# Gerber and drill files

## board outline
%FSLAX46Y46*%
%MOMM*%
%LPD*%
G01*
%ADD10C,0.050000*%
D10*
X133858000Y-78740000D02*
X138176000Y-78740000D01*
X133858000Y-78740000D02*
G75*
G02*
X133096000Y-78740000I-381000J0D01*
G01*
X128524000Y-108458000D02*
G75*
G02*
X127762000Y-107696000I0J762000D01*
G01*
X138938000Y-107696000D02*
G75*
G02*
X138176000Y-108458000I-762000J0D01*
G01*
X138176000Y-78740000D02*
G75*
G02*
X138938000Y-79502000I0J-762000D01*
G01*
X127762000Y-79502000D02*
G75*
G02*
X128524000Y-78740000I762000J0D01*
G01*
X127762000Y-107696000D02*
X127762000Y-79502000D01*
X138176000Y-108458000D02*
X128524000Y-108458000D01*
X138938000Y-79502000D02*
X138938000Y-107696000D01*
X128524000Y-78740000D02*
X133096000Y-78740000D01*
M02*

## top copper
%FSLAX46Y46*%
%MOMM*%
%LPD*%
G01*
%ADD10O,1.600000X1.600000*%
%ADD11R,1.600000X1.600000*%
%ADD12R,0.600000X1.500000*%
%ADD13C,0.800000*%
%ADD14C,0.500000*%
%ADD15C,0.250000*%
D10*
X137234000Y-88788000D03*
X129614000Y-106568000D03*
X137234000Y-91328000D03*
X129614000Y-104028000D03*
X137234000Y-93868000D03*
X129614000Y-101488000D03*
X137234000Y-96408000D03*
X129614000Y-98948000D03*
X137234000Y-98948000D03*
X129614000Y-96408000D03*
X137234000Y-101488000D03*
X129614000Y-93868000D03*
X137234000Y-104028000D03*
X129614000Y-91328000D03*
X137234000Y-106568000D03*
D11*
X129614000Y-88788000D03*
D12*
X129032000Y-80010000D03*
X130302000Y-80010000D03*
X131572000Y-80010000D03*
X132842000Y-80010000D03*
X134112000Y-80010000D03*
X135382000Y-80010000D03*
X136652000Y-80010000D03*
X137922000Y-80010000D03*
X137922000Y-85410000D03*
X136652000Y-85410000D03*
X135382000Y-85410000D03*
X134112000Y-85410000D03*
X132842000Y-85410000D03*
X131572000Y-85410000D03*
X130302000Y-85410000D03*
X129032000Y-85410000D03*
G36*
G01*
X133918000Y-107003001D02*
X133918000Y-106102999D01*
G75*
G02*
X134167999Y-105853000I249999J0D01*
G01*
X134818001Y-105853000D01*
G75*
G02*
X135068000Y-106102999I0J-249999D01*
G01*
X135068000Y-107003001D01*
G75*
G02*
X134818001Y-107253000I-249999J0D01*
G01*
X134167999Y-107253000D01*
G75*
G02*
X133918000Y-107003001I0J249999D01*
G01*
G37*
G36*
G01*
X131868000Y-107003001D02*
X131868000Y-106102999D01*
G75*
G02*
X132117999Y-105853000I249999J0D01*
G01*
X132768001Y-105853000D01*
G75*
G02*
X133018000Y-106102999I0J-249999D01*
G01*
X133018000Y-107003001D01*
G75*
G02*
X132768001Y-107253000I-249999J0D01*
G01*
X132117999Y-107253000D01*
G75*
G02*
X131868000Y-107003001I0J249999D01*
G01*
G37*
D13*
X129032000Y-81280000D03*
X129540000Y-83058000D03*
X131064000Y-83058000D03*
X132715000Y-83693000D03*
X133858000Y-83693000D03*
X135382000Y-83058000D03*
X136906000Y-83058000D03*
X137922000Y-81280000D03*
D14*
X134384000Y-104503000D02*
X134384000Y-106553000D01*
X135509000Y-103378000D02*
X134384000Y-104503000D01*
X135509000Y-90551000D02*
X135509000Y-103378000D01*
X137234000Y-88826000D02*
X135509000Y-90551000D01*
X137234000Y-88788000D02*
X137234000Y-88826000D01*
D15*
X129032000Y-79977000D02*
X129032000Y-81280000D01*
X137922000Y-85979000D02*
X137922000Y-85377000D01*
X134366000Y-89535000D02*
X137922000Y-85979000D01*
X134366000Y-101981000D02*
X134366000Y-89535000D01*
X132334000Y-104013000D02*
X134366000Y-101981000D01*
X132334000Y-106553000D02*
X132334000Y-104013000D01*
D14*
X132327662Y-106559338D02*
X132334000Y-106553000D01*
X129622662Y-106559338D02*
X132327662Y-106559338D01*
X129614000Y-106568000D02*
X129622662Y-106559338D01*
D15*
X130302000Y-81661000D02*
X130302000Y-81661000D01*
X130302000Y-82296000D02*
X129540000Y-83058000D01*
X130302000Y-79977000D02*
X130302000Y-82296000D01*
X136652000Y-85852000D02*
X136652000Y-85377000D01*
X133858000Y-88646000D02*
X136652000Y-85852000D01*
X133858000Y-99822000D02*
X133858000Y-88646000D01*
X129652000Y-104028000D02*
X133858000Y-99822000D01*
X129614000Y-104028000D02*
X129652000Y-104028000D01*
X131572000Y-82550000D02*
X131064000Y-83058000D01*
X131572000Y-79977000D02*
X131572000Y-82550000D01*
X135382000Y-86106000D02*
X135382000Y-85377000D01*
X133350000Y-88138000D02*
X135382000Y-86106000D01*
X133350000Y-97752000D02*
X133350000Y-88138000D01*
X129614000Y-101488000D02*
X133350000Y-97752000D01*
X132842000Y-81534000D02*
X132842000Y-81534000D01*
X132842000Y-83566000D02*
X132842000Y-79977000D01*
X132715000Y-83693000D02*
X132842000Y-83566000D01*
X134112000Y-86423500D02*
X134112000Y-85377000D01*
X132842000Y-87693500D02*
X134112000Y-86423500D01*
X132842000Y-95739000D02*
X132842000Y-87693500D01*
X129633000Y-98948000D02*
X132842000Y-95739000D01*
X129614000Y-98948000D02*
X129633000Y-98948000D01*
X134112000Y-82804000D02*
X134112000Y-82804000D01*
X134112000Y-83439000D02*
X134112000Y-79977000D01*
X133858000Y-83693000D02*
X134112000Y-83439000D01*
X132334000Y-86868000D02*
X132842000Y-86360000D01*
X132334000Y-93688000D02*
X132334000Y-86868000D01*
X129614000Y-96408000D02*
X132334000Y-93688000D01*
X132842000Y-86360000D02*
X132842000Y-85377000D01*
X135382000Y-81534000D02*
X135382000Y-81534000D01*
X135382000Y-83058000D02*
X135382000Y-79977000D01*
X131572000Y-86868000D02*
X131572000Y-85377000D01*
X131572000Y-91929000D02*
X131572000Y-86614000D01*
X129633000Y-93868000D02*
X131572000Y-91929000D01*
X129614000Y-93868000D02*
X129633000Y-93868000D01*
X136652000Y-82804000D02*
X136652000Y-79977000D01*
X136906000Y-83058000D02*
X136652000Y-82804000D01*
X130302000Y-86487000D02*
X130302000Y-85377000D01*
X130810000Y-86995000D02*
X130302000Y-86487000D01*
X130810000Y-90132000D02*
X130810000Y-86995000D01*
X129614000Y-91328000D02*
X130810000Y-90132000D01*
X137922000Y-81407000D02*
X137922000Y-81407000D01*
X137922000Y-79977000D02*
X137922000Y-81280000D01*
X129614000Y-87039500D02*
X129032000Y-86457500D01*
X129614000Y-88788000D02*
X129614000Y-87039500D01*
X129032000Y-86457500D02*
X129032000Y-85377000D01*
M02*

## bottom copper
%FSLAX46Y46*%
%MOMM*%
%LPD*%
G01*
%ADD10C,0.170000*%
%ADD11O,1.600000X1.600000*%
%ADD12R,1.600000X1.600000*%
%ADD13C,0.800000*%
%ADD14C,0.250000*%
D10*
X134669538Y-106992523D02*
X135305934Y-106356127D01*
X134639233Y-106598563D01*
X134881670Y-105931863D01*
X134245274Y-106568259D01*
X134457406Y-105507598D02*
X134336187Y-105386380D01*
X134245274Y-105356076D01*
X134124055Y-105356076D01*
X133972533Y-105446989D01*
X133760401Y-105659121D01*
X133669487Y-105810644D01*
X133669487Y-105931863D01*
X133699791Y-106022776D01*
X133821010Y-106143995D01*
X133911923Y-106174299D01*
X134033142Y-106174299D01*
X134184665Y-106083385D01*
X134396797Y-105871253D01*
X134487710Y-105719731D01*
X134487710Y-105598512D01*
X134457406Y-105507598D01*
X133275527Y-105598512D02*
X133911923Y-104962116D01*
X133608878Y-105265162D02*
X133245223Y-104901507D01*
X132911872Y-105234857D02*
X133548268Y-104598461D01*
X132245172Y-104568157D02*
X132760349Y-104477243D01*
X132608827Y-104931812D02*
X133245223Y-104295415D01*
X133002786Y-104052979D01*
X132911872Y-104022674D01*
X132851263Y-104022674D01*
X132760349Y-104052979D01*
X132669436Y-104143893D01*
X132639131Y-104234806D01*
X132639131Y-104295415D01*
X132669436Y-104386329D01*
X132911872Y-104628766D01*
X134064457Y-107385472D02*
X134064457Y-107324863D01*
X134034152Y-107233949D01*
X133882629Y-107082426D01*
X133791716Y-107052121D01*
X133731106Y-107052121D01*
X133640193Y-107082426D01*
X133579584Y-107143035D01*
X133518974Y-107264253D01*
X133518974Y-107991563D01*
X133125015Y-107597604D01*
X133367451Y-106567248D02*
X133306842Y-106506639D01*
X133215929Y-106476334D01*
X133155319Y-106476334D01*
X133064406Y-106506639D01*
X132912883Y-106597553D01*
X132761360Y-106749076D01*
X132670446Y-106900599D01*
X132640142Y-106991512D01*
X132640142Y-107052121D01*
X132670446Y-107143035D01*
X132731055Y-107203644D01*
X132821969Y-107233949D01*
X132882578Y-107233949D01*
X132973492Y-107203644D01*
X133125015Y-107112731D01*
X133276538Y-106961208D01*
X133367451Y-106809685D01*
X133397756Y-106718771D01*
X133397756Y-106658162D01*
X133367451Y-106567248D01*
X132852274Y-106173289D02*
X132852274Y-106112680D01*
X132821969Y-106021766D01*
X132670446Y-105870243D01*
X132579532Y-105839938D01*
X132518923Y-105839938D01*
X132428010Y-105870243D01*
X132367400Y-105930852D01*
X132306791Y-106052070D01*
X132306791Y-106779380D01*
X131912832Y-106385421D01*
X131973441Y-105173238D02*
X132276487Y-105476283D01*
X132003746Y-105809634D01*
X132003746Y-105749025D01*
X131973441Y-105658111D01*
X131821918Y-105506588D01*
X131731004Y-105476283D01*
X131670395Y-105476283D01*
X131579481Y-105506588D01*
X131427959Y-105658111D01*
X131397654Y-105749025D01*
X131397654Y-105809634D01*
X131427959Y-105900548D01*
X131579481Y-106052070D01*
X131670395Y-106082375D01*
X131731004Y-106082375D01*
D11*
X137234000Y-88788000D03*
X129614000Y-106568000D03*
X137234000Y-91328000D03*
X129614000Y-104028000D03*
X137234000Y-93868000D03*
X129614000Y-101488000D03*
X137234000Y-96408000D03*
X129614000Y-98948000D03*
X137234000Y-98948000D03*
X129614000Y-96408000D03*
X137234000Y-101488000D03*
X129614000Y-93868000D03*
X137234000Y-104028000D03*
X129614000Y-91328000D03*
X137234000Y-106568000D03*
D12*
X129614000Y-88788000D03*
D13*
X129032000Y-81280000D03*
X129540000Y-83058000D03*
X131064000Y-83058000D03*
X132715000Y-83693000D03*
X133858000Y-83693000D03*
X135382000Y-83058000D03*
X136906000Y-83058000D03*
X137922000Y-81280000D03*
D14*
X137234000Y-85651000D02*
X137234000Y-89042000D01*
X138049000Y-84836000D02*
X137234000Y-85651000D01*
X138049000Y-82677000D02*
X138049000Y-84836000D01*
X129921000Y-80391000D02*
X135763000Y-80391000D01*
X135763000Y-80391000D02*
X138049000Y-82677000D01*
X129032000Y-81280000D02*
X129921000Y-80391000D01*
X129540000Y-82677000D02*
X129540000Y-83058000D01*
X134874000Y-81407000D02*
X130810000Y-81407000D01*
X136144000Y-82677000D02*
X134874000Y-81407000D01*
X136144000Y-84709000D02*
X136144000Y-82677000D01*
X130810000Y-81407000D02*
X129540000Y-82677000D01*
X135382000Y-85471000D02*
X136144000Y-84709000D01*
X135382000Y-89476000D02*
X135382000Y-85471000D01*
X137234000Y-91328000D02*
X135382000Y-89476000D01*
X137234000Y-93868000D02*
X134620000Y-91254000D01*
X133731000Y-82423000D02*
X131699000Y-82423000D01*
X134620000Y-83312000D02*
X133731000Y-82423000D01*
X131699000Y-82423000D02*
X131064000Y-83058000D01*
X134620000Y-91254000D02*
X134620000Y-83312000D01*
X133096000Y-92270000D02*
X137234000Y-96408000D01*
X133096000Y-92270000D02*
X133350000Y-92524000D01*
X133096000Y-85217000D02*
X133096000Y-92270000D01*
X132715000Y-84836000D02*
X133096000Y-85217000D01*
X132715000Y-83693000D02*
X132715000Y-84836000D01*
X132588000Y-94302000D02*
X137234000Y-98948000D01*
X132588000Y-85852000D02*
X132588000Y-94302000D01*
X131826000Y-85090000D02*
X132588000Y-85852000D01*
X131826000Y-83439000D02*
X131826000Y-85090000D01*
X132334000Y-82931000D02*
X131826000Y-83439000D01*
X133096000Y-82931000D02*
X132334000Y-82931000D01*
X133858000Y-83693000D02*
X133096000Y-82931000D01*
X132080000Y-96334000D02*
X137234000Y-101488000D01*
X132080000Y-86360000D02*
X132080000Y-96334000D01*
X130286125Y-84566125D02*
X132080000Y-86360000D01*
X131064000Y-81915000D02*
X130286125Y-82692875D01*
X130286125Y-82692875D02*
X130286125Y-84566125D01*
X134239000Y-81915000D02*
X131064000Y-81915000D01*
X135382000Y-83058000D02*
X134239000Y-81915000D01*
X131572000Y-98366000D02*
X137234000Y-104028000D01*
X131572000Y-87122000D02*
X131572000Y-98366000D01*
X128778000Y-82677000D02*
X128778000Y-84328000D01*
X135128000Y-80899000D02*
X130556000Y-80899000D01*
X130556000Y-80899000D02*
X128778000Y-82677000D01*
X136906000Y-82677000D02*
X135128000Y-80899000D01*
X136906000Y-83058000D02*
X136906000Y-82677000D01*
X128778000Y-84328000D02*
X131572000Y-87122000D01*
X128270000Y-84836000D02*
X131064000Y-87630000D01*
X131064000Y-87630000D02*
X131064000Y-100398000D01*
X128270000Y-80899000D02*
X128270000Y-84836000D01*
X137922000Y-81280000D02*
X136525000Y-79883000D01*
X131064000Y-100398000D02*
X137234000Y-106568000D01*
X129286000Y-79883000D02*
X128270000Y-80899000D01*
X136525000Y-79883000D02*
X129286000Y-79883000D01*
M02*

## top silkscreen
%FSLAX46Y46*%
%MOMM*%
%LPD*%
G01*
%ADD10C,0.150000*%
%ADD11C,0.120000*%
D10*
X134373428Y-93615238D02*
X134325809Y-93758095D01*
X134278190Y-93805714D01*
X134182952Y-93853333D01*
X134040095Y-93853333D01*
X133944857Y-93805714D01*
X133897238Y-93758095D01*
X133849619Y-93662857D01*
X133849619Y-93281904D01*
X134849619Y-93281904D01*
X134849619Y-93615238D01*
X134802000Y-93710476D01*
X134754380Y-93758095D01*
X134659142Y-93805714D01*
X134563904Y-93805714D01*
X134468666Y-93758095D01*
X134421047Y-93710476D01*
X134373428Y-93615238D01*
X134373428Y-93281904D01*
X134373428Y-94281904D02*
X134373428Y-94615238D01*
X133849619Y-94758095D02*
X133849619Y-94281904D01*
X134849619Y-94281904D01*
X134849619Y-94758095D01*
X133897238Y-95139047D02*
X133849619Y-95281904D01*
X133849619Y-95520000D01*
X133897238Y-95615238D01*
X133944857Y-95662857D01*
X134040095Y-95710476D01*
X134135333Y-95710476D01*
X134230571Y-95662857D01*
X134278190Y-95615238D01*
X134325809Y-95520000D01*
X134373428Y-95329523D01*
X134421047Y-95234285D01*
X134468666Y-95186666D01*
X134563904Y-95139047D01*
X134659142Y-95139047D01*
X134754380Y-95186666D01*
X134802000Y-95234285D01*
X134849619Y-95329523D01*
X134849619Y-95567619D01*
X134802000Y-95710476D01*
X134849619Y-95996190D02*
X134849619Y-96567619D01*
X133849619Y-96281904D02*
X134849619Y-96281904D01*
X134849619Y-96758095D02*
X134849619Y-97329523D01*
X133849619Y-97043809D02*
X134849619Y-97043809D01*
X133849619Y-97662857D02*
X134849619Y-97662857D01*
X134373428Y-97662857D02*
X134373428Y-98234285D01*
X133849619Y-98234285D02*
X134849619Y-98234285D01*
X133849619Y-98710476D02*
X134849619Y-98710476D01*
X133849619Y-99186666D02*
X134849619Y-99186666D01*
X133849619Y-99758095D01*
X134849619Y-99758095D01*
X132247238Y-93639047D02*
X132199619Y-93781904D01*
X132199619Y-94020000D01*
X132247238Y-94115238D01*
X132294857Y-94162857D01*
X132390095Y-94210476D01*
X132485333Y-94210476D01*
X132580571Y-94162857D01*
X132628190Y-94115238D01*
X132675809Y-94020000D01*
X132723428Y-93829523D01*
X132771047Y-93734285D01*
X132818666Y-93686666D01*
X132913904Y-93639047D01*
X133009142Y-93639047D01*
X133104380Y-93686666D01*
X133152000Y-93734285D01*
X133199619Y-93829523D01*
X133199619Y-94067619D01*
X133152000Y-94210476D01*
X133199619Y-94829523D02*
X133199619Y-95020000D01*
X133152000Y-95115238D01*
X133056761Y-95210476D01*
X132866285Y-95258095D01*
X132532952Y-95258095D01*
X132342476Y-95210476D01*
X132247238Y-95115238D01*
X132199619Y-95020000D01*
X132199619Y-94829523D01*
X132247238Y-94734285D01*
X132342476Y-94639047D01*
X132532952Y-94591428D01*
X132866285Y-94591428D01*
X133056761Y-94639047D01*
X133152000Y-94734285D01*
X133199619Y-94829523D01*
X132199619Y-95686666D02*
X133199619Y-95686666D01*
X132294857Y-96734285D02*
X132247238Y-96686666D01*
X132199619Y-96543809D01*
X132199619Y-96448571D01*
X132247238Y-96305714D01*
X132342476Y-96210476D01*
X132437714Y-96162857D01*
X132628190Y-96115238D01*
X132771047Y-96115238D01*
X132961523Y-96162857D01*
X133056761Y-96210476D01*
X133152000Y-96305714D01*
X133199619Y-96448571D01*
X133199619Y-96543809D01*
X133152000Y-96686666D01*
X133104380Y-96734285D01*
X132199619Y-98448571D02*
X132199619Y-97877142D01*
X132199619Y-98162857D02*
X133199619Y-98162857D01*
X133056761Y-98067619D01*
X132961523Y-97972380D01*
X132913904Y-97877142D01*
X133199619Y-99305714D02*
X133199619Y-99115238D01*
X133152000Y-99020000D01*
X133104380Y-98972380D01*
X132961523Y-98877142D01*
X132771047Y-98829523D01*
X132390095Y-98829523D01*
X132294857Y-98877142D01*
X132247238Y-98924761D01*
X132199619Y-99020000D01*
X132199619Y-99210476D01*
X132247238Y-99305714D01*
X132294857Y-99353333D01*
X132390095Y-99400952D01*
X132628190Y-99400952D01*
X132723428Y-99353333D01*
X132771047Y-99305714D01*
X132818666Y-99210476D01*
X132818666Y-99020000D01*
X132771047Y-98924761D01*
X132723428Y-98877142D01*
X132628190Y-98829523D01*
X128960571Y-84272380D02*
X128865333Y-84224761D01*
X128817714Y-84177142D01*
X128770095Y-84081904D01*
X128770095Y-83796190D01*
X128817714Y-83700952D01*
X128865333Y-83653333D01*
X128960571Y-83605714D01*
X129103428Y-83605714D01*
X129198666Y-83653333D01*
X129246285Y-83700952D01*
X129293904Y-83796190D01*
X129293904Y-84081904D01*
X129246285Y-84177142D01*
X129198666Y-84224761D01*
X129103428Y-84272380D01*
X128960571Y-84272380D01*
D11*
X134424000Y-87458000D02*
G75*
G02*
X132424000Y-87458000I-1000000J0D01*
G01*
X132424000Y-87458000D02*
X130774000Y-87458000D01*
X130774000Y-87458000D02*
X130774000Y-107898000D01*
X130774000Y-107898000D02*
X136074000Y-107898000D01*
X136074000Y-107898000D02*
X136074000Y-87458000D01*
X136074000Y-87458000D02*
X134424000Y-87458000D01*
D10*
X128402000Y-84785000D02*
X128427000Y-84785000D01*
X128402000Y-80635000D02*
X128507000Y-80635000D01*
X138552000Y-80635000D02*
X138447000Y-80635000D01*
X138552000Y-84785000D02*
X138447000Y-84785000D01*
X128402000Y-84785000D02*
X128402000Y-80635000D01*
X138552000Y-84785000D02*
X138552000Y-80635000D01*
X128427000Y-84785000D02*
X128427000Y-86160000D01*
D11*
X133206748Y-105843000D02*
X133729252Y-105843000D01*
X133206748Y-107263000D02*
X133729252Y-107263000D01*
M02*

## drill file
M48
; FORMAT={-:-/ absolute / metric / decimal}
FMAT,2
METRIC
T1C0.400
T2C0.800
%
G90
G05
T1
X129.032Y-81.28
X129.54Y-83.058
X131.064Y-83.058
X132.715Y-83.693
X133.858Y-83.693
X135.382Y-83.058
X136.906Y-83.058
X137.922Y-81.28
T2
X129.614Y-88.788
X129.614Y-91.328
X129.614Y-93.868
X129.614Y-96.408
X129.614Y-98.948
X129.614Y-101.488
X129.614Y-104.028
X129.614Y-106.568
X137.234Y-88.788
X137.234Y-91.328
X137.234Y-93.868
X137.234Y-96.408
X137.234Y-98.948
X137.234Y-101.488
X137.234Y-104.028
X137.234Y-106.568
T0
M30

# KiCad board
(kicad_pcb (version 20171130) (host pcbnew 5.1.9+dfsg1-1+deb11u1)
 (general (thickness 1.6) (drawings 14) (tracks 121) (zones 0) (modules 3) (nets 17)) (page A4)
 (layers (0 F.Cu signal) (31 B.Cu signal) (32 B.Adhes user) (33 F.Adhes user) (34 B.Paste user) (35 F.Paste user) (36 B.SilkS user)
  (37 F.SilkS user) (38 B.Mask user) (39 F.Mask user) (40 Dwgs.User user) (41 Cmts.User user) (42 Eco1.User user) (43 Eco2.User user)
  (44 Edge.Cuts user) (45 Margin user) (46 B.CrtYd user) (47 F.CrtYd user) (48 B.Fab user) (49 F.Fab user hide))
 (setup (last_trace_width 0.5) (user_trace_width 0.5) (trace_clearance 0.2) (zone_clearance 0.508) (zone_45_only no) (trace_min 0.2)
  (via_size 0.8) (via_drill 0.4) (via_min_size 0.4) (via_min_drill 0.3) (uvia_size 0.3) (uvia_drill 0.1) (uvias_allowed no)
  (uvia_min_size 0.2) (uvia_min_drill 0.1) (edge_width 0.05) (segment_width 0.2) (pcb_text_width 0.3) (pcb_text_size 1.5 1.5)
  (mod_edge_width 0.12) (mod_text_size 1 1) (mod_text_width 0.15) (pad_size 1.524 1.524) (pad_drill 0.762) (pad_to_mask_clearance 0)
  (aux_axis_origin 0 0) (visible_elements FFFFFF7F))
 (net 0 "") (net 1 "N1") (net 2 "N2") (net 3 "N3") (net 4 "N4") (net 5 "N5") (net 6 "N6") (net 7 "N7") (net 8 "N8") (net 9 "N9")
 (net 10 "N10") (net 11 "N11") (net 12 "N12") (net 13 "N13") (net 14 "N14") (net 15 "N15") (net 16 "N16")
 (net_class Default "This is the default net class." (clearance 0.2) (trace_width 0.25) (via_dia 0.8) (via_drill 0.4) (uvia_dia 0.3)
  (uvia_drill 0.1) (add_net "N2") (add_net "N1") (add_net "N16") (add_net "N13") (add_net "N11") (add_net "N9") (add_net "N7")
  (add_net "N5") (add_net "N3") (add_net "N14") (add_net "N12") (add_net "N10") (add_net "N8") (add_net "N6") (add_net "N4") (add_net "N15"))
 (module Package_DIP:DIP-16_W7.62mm (layer F.Cu) (at 129.614 88.788)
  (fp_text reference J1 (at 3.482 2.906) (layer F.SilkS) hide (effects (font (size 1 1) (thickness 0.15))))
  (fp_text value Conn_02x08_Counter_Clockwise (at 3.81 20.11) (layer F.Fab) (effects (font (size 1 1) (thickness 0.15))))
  (fp_arc (start 3.81 -1.33) (end 2.81 -1.33) (angle -180) (layer F.SilkS) (width 0.12))
  (fp_line (start 2.81 -1.33) (end 1.16 -1.33) (layer F.SilkS) (width 0.12))
  (fp_line (start 1.16 -1.33) (end 1.16 19.11) (layer F.SilkS) (width 0.12))
  (fp_line (start 1.16 19.11) (end 6.46 19.11) (layer F.SilkS) (width 0.12))
  (fp_line (start 6.46 19.11) (end 6.46 -1.33) (layer F.SilkS) (width 0.12))
  (fp_line (start 6.46 -1.33) (end 4.81 -1.33) (layer F.SilkS) (width 0.12))
  (pad 16 thru_hole oval (at 7.62 0) (size 1.6 1.6) (drill 0.8) (layers *.Cu *.Mask) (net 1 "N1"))
  (pad 8 thru_hole oval (at 0 17.78) (size 1.6 1.6) (drill 0.8) (layers *.Cu *.Mask) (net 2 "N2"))
  (pad 15 thru_hole oval (at 7.62 2.54) (size 1.6 1.6) (drill 0.8) (layers *.Cu *.Mask) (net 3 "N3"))
  (pad 7 thru_hole oval (at 0 15.24) (size 1.6 1.6) (drill 0.8) (layers *.Cu *.Mask) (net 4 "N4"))
  (pad 14 thru_hole oval (at 7.62 5.08) (size 1.6 1.6) (drill 0.8) (layers *.Cu *.Mask) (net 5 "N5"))
  (pad 6 thru_hole oval (at 0 12.7) (size 1.6 1.6) (drill 0.8) (layers *.Cu *.Mask) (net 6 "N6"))
  (pad 13 thru_hole oval (at 7.62 7.62) (size 1.6 1.6) (drill 0.8) (layers *.Cu *.Mask) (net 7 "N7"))
  (pad 5 thru_hole oval (at 0 10.16) (size 1.6 1.6) (drill 0.8) (layers *.Cu *.Mask) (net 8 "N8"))
  (pad 12 thru_hole oval (at 7.62 10.16) (size 1.6 1.6) (drill 0.8) (layers *.Cu *.Mask) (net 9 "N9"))
  (pad 4 thru_hole oval (at 0 7.62) (size 1.6 1.6) (drill 0.8) (layers *.Cu *.Mask) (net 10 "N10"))
  (pad 11 thru_hole oval (at 7.62 12.7) (size 1.6 1.6) (drill 0.8) (layers *.Cu *.Mask) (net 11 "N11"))
  (pad 3 thru_hole oval (at 0 5.08) (size 1.6 1.6) (drill 0.8) (layers *.Cu *.Mask) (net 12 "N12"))
  (pad 10 thru_hole oval (at 7.62 15.24) (size 1.6 1.6) (drill 0.8) (layers *.Cu *.Mask) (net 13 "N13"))
  (pad 2 thru_hole oval (at 0 2.54) (size 1.6 1.6) (drill 0.8) (layers *.Cu *.Mask) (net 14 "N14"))
  (pad 9 thru_hole oval (at 7.62 17.78) (size 1.6 1.6) (drill 0.8) (layers *.Cu *.Mask) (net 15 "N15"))
  (pad 1 thru_hole rect (at 0 0) (size 1.6 1.6) (drill 0.8) (layers *.Cu *.Mask) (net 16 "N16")))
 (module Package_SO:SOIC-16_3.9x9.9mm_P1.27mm (layer F.Cu) (at 133.477 82.71 90)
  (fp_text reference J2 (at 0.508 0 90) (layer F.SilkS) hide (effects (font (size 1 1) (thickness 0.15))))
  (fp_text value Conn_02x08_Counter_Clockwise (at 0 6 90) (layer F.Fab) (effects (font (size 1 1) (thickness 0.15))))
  (fp_line (start -2.075 -5.075) (end -2.075 -5.05) (layer F.SilkS) (width 0.15))
  (fp_line (start 2.075 -5.075) (end 2.075 -4.97) (layer F.SilkS) (width 0.15))
  (fp_line (start 2.075 5.075) (end 2.075 4.97) (layer F.SilkS) (width 0.15))
  (fp_line (start -2.075 5.075) (end -2.075 4.97) (layer F.SilkS) (width 0.15))
  (fp_line (start -2.075 -5.075) (end 2.075 -5.075) (layer F.SilkS) (width 0.15))
  (fp_line (start -2.075 5.075) (end 2.075 5.075) (layer F.SilkS) (width 0.15))
  (fp_line (start -2.075 -5.05) (end -3.45 -5.05) (layer F.SilkS) (width 0.15))
  (pad 16 smd rect (at 2.7 -4.445 90) (size 1.5 0.6) (layers F.Cu F.Paste F.Mask) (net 1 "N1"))
  (pad 15 smd rect (at 2.7 -3.175 90) (size 1.5 0.6) (layers F.Cu F.Paste F.Mask) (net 3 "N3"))
  (pad 14 smd rect (at 2.7 -1.905 90) (size 1.5 0.6) (layers F.Cu F.Paste F.Mask) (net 5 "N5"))
  (pad 13 smd rect (at 2.7 -0.635 90) (size 1.5 0.6) (layers F.Cu F.Paste F.Mask) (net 7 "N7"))
  (pad 12 smd rect (at 2.7 0.635 90) (size 1.5 0.6) (layers F.Cu F.Paste F.Mask) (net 9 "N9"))
  (pad 11 smd rect (at 2.7 1.905 90) (size 1.5 0.6) (layers F.Cu F.Paste F.Mask) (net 11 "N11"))
  (pad 10 smd rect (at 2.7 3.175 90) (size 1.5 0.6) (layers F.Cu F.Paste F.Mask) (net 13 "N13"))
  (pad 9 smd rect (at 2.7 4.445 90) (size 1.5 0.6) (layers F.Cu F.Paste F.Mask) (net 15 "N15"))
  (pad 8 smd rect (at -2.7 4.445 90) (size 1.5 0.6) (layers F.Cu F.Paste F.Mask) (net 2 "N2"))
  (pad 7 smd rect (at -2.7 3.175 90) (size 1.5 0.6) (layers F.Cu F.Paste F.Mask) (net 4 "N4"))
  (pad 6 smd rect (at -2.7 1.905 90) (size 1.5 0.6) (layers F.Cu F.Paste F.Mask) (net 6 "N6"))
  (pad 5 smd rect (at -2.7 0.635 90) (size 1.5 0.6) (layers F.Cu F.Paste F.Mask) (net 8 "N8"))
  (pad 4 smd rect (at -2.7 -0.635 90) (size 1.5 0.6) (layers F.Cu F.Paste F.Mask) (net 10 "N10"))
  (pad 3 smd rect (at -2.7 -1.905 90) (size 1.5 0.6) (layers F.Cu F.Paste F.Mask) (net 12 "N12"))
  (pad 2 smd rect (at -2.7 -3.175 90) (size 1.5 0.6) (layers F.Cu F.Paste F.Mask) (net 14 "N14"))
  (pad 1 smd rect (at -2.7 -4.445 90) (size 1.5 0.6) (layers F.Cu F.Paste F.Mask) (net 16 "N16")))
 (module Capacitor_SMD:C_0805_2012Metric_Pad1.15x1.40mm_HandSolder (layer F.Cu) (at 133.468 106.553)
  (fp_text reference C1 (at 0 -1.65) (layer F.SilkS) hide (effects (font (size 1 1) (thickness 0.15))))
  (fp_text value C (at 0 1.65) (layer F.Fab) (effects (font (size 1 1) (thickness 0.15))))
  (fp_line (start -0.261252 -0.71) (end 0.261252 -0.71) (layer F.SilkS) (width 0.12))
  (fp_line (start -0.261252 0.71) (end 0.261252 0.71) (layer F.SilkS) (width 0.12))
  (pad 2 smd roundrect (at 1.025 0) (size 1.15 1.4) (layers F.Cu F.Paste F.Mask) (roundrect_rratio 0.2173904347826087) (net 1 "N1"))
  (pad 1 smd roundrect (at -1.025 0) (size 1.15 1.4) (layers F.Cu F.Paste F.Mask) (roundrect_rratio 0.2173904347826087) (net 2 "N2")))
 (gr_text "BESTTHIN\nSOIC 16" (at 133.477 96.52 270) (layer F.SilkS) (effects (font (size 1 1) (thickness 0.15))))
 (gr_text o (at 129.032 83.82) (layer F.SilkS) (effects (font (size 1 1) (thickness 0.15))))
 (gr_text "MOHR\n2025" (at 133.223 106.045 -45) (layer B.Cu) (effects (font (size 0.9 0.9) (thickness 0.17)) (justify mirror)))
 (gr_line (start 133.858 78.74) (end 138.176 78.74) (layer Edge.Cuts) (width 0.05))
 (gr_arc (start 133.477 78.74) (end 133.096 78.74) (angle -180) (layer Edge.Cuts) (width 0.05))
 (gr_arc (start 128.524 107.696) (end 127.762 107.696) (angle -90) (layer Edge.Cuts) (width 0.05))
 (gr_arc (start 138.176 107.696) (end 138.176 108.458) (angle -90) (layer Edge.Cuts) (width 0.05))
 (gr_arc (start 138.176 79.502) (end 138.938 79.502) (angle -90) (layer Edge.Cuts) (width 0.05))
 (gr_arc (start 128.524 79.502) (end 128.524 78.74) (angle -90) (layer Edge.Cuts) (width 0.05))
 (gr_line (start 127.762 107.696) (end 127.762 79.502) (layer Edge.Cuts) (width 0.05))
 (gr_line (start 138.176 108.458) (end 128.524 108.458) (layer Edge.Cuts) (width 0.05))
 (gr_line (start 138.938 79.502) (end 138.938 107.696) (layer Edge.Cuts) (width 0.05))
 (gr_line (start 128.524 78.74) (end 133.096 78.74) (layer Edge.Cuts) (width 0.05))
 (segment (start 134.384 104.503) (end 134.384 106.553) (width 0.5) (layer F.Cu) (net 1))
 (segment (start 135.509 103.378) (end 134.384 104.503) (width 0.5) (layer F.Cu) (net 1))
 (segment (start 135.509 90.551) (end 135.509 103.378) (width 0.5) (layer F.Cu) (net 1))
 (segment (start 137.234 88.826) (end 135.509 90.551) (width 0.5) (layer F.Cu) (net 1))
 (segment (start 137.234 88.788) (end 137.234 88.826) (width 0.5) (layer F.Cu) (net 1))
 (segment (start 137.234 85.651) (end 137.234 89.042) (width 0.25) (layer B.Cu) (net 1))
 (segment (start 138.049 84.836) (end 137.234 85.651) (width 0.25) (layer B.Cu) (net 1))
 (segment (start 138.049 82.677) (end 138.049 84.836) (width 0.25) (layer B.Cu) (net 1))
 (segment (start 129.921 80.391) (end 135.763 80.391) (width 0.25) (layer B.Cu) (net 1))
 (segment (start 135.763 80.391) (end 138.049 82.677) (width 0.25) (layer B.Cu) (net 1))
 (segment (start 129.032 81.28) (end 129.921 80.391) (width 0.25) (layer B.Cu) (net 1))
 (segment (start 129.032 79.977) (end 129.032 81.28) (width 0.25) (layer F.Cu) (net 1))
 (via (at 129.032 81.28) (size 0.8) (drill 0.4) (layers F.Cu B.Cu) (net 1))
 (segment (start 137.922 85.979) (end 137.922 85.377) (width 0.25) (layer F.Cu) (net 2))
 (segment (start 134.366 89.535) (end 137.922 85.979) (width 0.25) (layer F.Cu) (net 2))
 (segment (start 134.366 101.981) (end 134.366 89.535) (width 0.25) (layer F.Cu) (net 2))
 (segment (start 132.334 104.013) (end 134.366 101.981) (width 0.25) (layer F.Cu) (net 2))
 (segment (start 132.334 106.553) (end 132.334 104.013) (width 0.25) (layer F.Cu) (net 2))
 (segment (start 132.327662 106.559338) (end 132.334 106.553) (width 0.5) (layer F.Cu) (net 2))
 (segment (start 129.622662 106.559338) (end 132.327662 106.559338) (width 0.5) (layer F.Cu) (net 2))
 (segment (start 129.614 106.568) (end 129.622662 106.559338) (width 0.5) (layer F.Cu) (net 2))
 (segment (start 130.302 81.661) (end 130.302 81.661) (width 0.25) (layer F.Cu) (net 3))
 (segment (start 130.302 82.296) (end 129.54 83.058) (width 0.25) (layer F.Cu) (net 3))
 (segment (start 130.302 79.977) (end 130.302 82.296) (width 0.25) (layer F.Cu) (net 3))
 (via (at 129.54 83.058) (size 0.8) (drill 0.4) (layers F.Cu B.Cu) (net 3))
 (segment (start 129.54 82.677) (end 129.54 83.058) (width 0.25) (layer B.Cu) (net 3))
 (segment (start 134.874 81.407) (end 130.81 81.407) (width 0.25) (layer B.Cu) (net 3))
 (segment (start 136.144 82.677) (end 134.874 81.407) (width 0.25) (layer B.Cu) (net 3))
 (segment (start 136.144 84.709) (end 136.144 82.677) (width 0.25) (layer B.Cu) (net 3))
 (segment (start 130.81 81.407) (end 129.54 82.677) (width 0.25) (layer B.Cu) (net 3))
 (segment (start 135.382 85.471) (end 136.144 84.709) (width 0.25) (layer B.Cu) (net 3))
 (segment (start 135.382 89.476) (end 135.382 85.471) (width 0.25) (layer B.Cu) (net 3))
 (segment (start 137.234 91.328) (end 135.382 89.476) (width 0.25) (layer B.Cu) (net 3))
 (segment (start 136.652 85.852) (end 136.652 85.377) (width 0.25) (layer F.Cu) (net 4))
 (segment (start 133.858 88.646) (end 136.652 85.852) (width 0.25) (layer F.Cu) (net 4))
 (segment (start 133.858 99.822) (end 133.858 88.646) (width 0.25) (layer F.Cu) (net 4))
 (segment (start 129.652 104.028) (end 133.858 99.822) (width 0.25) (layer F.Cu) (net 4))
 (segment (start 129.614 104.028) (end 129.652 104.028) (width 0.25) (layer F.Cu) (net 4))
 (segment (start 131.572 82.55) (end 131.064 83.058) (width 0.25) (layer F.Cu) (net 5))
 (segment (start 131.572 79.977) (end 131.572 82.55) (width 0.25) (layer F.Cu) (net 5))
 (via (at 131.064 83.058) (size 0.8) (drill 0.4) (layers F.Cu B.Cu) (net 5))
 (segment (start 137.234 93.868) (end 134.62 91.254) (width 0.25) (layer B.Cu) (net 5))
 (segment (start 133.731 82.423) (end 131.699 82.423) (width 0.25) (layer B.Cu) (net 5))
 (segment (start 134.62 83.312) (end 133.731 82.423) (width 0.25) (layer B.Cu) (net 5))
 (segment (start 131.699 82.423) (end 131.064 83.058) (width 0.25) (layer B.Cu) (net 5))
 (segment (start 134.62 91.254) (end 134.62 83.312) (width 0.25) (layer B.Cu) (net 5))
 (segment (start 135.382 86.106) (end 135.382 85.377) (width 0.25) (layer F.Cu) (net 6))
 (segment (start 133.35 88.138) (end 135.382 86.106) (width 0.25) (layer F.Cu) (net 6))
 (segment (start 133.35 97.752) (end 133.35 88.138) (width 0.25) (layer F.Cu) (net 6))
 (segment (start 129.614 101.488) (end 133.35 97.752) (width 0.25) (layer F.Cu) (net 6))
 (segment (start 132.842 81.534) (end 132.842 81.534) (width 0.25) (layer F.Cu) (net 7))
 (segment (start 132.842 83.566) (end 132.842 79.977) (width 0.25) (layer F.Cu) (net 7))
 (segment (start 132.715 83.693) (end 132.842 83.566) (width 0.25) (layer F.Cu) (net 7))
 (via (at 132.715 83.693) (size 0.8) (drill 0.4) (layers F.Cu B.Cu) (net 7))
 (segment (start 133.096 92.27) (end 137.234 96.408) (width 0.25) (layer B.Cu) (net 7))
 (segment (start 133.096 92.27) (end 133.35 92.524) (width 0.25) (layer B.Cu) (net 7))
 (segment (start 133.096 85.217) (end 133.096 92.27) (width 0.25) (layer B.Cu) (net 7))
 (segment (start 132.715 84.836) (end 133.096 85.217) (width 0.25) (layer B.Cu) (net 7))
 (segment (start 132.715 83.693) (end 132.715 84.836) (width 0.25) (layer B.Cu) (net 7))
 (segment (start 134.112 86.4235) (end 134.112 85.377) (width 0.25) (layer F.Cu) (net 8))
 (segment (start 132.842 87.6935) (end 134.112 86.4235) (width 0.25) (layer F.Cu) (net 8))
 (segment (start 132.842 95.739) (end 132.842 87.6935) (width 0.25) (layer F.Cu) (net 8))
 (segment (start 129.633 98.948) (end 132.842 95.739) (width 0.25) (layer F.Cu) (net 8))
 (segment (start 129.614 98.948) (end 129.633 98.948) (width 0.25) (layer F.Cu) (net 8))
 (segment (start 134.112 82.804) (end 134.112 82.804) (width 0.25) (layer F.Cu) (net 9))
 (segment (start 134.112 83.439) (end 134.112 79.977) (width 0.25) (layer F.Cu) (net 9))
 (segment (start 133.858 83.693) (end 134.112 83.439) (width 0.25) (layer F.Cu) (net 9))
 (via (at 133.858 83.693) (size 0.8) (drill 0.4) (layers F.Cu B.Cu) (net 9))
 (segment (start 132.588 94.302) (end 137.234 98.948) (width 0.25) (layer B.Cu) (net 9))
 (segment (start 132.588 85.852) (end 132.588 94.302) (width 0.25) (layer B.Cu) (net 9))
 (segment (start 131.826 85.09) (end 132.588 85.852) (width 0.25) (layer B.Cu) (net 9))
 (segment (start 131.826 83.439) (end 131.826 85.09) (width 0.25) (layer B.Cu) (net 9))
 (segment (start 132.334 82.931) (end 131.826 83.439) (width 0.25) (layer B.Cu) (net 9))
 (segment (start 133.096 82.931) (end 132.334 82.931) (width 0.25) (layer B.Cu) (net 9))
 (segment (start 133.858 83.693) (end 133.096 82.931) (width 0.25) (layer B.Cu) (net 9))
 (segment (start 132.334 86.868) (end 132.842 86.36) (width 0.25) (layer F.Cu) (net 10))
 (segment (start 132.334 93.688) (end 132.334 86.868) (width 0.25) (layer F.Cu) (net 10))
 (segment (start 129.614 96.408) (end 132.334 93.688) (width 0.25) (layer F.Cu) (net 10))
 (segment (start 132.842 86.36) (end 132.842 85.377) (width 0.25) (layer F.Cu) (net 10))
 (segment (start 135.382 81.534) (end 135.382 81.534) (width 0.25) (layer F.Cu) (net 11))
 (segment (start 135.382 83.058) (end 135.382 79.977) (width 0.25) (layer F.Cu) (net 11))
 (via (at 135.382 83.058) (size 0.8) (drill 0.4) (layers F.Cu B.Cu) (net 11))
 (segment (start 132.08 96.334) (end 137.234 101.488) (width 0.25) (layer B.Cu) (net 11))
 (segment (start 132.08 86.36) (end 132.08 96.334) (width 0.25) (layer B.Cu) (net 11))
 (segment (start 130.286125 84.566125) (end 132.08 86.36) (width 0.25) (layer B.Cu) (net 11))
 (segment (start 131.064 81.915) (end 130.286125 82.692875) (width 0.25) (layer B.Cu) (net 11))
 (segment (start 130.286125 82.692875) (end 130.286125 84.566125) (width 0.25) (layer B.Cu) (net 11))
 (segment (start 134.239 81.915) (end 131.064 81.915) (width 0.25) (layer B.Cu) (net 11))
 (segment (start 135.382 83.058) (end 134.239 81.915) (width 0.25) (layer B.Cu) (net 11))
 (segment (start 131.572 86.868) (end 131.572 85.377) (width 0.25) (layer F.Cu) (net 12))
 (segment (start 131.572 91.929) (end 131.572 86.614) (width 0.25) (layer F.Cu) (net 12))
 (segment (start 129.633 93.868) (end 131.572 91.929) (width 0.25) (layer F.Cu) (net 12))
 (segment (start 129.614 93.868) (end 129.633 93.868) (width 0.25) (layer F.Cu) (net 12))
 (segment (start 131.572 98.366) (end 137.234 104.028) (width 0.25) (layer B.Cu) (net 13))
 (segment (start 131.572 87.122) (end 131.572 98.366) (width 0.25) (layer B.Cu) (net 13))
 (segment (start 128.778 82.677) (end 128.778 84.328) (width 0.25) (layer B.Cu) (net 13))
 (segment (start 135.128 80.899) (end 130.556 80.899) (width 0.25) (layer B.Cu) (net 13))
 (segment (start 130.556 80.899) (end 128.778 82.677) (width 0.25) (layer B.Cu) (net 13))
 (segment (start 136.906 82.677) (end 135.128 80.899) (width 0.25) (layer B.Cu) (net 13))
 (segment (start 136.906 83.058) (end 136.906 82.677) (width 0.25) (layer B.Cu) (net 13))
 (segment (start 136.652 82.804) (end 136.652 79.977) (width 0.25) (layer F.Cu) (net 13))
 (segment (start 136.906 83.058) (end 136.652 82.804) (width 0.25) (layer F.Cu) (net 13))
 (segment (start 128.778 84.328) (end 131.572 87.122) (width 0.25) (layer B.Cu) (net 13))
 (via (at 136.906 83.058) (size 0.8) (drill 0.4) (layers F.Cu B.Cu) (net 13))
 (segment (start 130.302 86.487) (end 130.302 85.377) (width 0.25) (layer F.Cu) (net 14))
 (segment (start 130.81 86.995) (end 130.302 86.487) (width 0.25) (layer F.Cu) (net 14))
 (segment (start 130.81 90.132) (end 130.81 86.995) (width 0.25) (layer F.Cu) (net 14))
 (segment (start 129.614 91.328) (end 130.81 90.132) (width 0.25) (layer F.Cu) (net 14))
 (segment (start 137.922 81.407) (end 137.922 81.407) (width 0.25) (layer F.Cu) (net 15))
 (segment (start 128.27 84.836) (end 131.064 87.63) (width 0.25) (layer B.Cu) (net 15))
 (segment (start 131.064 87.63) (end 131.064 100.398) (width 0.25) (layer B.Cu) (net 15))
 (segment (start 128.27 80.899) (end 128.27 84.836) (width 0.25) (layer B.Cu) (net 15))
 (segment (start 137.922 81.28) (end 136.525 79.883) (width 0.25) (layer B.Cu) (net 15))
 (segment (start 131.064 100.398) (end 137.234 106.568) (width 0.25) (layer B.Cu) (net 15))
 (segment (start 137.922 79.977) (end 137.922 81.28) (width 0.25) (layer F.Cu) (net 15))
 (segment (start 129.286 79.883) (end 128.27 80.899) (width 0.25) (layer B.Cu) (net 15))
 (segment (start 136.525 79.883) (end 129.286 79.883) (width 0.25) (layer B.Cu) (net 15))
 (via (at 137.922 81.28) (size 0.8) (drill 0.4) (layers F.Cu B.Cu) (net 15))
 (segment (start 129.614 87.0395) (end 129.032 86.4575) (width 0.25) (layer F.Cu) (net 16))
 (segment (start 129.614 88.788) (end 129.614 87.0395) (width 0.25) (layer F.Cu) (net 16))
 (segment (start 129.032 86.4575) (end 129.032 85.377) (width 0.25) (layer F.Cu) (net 16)))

